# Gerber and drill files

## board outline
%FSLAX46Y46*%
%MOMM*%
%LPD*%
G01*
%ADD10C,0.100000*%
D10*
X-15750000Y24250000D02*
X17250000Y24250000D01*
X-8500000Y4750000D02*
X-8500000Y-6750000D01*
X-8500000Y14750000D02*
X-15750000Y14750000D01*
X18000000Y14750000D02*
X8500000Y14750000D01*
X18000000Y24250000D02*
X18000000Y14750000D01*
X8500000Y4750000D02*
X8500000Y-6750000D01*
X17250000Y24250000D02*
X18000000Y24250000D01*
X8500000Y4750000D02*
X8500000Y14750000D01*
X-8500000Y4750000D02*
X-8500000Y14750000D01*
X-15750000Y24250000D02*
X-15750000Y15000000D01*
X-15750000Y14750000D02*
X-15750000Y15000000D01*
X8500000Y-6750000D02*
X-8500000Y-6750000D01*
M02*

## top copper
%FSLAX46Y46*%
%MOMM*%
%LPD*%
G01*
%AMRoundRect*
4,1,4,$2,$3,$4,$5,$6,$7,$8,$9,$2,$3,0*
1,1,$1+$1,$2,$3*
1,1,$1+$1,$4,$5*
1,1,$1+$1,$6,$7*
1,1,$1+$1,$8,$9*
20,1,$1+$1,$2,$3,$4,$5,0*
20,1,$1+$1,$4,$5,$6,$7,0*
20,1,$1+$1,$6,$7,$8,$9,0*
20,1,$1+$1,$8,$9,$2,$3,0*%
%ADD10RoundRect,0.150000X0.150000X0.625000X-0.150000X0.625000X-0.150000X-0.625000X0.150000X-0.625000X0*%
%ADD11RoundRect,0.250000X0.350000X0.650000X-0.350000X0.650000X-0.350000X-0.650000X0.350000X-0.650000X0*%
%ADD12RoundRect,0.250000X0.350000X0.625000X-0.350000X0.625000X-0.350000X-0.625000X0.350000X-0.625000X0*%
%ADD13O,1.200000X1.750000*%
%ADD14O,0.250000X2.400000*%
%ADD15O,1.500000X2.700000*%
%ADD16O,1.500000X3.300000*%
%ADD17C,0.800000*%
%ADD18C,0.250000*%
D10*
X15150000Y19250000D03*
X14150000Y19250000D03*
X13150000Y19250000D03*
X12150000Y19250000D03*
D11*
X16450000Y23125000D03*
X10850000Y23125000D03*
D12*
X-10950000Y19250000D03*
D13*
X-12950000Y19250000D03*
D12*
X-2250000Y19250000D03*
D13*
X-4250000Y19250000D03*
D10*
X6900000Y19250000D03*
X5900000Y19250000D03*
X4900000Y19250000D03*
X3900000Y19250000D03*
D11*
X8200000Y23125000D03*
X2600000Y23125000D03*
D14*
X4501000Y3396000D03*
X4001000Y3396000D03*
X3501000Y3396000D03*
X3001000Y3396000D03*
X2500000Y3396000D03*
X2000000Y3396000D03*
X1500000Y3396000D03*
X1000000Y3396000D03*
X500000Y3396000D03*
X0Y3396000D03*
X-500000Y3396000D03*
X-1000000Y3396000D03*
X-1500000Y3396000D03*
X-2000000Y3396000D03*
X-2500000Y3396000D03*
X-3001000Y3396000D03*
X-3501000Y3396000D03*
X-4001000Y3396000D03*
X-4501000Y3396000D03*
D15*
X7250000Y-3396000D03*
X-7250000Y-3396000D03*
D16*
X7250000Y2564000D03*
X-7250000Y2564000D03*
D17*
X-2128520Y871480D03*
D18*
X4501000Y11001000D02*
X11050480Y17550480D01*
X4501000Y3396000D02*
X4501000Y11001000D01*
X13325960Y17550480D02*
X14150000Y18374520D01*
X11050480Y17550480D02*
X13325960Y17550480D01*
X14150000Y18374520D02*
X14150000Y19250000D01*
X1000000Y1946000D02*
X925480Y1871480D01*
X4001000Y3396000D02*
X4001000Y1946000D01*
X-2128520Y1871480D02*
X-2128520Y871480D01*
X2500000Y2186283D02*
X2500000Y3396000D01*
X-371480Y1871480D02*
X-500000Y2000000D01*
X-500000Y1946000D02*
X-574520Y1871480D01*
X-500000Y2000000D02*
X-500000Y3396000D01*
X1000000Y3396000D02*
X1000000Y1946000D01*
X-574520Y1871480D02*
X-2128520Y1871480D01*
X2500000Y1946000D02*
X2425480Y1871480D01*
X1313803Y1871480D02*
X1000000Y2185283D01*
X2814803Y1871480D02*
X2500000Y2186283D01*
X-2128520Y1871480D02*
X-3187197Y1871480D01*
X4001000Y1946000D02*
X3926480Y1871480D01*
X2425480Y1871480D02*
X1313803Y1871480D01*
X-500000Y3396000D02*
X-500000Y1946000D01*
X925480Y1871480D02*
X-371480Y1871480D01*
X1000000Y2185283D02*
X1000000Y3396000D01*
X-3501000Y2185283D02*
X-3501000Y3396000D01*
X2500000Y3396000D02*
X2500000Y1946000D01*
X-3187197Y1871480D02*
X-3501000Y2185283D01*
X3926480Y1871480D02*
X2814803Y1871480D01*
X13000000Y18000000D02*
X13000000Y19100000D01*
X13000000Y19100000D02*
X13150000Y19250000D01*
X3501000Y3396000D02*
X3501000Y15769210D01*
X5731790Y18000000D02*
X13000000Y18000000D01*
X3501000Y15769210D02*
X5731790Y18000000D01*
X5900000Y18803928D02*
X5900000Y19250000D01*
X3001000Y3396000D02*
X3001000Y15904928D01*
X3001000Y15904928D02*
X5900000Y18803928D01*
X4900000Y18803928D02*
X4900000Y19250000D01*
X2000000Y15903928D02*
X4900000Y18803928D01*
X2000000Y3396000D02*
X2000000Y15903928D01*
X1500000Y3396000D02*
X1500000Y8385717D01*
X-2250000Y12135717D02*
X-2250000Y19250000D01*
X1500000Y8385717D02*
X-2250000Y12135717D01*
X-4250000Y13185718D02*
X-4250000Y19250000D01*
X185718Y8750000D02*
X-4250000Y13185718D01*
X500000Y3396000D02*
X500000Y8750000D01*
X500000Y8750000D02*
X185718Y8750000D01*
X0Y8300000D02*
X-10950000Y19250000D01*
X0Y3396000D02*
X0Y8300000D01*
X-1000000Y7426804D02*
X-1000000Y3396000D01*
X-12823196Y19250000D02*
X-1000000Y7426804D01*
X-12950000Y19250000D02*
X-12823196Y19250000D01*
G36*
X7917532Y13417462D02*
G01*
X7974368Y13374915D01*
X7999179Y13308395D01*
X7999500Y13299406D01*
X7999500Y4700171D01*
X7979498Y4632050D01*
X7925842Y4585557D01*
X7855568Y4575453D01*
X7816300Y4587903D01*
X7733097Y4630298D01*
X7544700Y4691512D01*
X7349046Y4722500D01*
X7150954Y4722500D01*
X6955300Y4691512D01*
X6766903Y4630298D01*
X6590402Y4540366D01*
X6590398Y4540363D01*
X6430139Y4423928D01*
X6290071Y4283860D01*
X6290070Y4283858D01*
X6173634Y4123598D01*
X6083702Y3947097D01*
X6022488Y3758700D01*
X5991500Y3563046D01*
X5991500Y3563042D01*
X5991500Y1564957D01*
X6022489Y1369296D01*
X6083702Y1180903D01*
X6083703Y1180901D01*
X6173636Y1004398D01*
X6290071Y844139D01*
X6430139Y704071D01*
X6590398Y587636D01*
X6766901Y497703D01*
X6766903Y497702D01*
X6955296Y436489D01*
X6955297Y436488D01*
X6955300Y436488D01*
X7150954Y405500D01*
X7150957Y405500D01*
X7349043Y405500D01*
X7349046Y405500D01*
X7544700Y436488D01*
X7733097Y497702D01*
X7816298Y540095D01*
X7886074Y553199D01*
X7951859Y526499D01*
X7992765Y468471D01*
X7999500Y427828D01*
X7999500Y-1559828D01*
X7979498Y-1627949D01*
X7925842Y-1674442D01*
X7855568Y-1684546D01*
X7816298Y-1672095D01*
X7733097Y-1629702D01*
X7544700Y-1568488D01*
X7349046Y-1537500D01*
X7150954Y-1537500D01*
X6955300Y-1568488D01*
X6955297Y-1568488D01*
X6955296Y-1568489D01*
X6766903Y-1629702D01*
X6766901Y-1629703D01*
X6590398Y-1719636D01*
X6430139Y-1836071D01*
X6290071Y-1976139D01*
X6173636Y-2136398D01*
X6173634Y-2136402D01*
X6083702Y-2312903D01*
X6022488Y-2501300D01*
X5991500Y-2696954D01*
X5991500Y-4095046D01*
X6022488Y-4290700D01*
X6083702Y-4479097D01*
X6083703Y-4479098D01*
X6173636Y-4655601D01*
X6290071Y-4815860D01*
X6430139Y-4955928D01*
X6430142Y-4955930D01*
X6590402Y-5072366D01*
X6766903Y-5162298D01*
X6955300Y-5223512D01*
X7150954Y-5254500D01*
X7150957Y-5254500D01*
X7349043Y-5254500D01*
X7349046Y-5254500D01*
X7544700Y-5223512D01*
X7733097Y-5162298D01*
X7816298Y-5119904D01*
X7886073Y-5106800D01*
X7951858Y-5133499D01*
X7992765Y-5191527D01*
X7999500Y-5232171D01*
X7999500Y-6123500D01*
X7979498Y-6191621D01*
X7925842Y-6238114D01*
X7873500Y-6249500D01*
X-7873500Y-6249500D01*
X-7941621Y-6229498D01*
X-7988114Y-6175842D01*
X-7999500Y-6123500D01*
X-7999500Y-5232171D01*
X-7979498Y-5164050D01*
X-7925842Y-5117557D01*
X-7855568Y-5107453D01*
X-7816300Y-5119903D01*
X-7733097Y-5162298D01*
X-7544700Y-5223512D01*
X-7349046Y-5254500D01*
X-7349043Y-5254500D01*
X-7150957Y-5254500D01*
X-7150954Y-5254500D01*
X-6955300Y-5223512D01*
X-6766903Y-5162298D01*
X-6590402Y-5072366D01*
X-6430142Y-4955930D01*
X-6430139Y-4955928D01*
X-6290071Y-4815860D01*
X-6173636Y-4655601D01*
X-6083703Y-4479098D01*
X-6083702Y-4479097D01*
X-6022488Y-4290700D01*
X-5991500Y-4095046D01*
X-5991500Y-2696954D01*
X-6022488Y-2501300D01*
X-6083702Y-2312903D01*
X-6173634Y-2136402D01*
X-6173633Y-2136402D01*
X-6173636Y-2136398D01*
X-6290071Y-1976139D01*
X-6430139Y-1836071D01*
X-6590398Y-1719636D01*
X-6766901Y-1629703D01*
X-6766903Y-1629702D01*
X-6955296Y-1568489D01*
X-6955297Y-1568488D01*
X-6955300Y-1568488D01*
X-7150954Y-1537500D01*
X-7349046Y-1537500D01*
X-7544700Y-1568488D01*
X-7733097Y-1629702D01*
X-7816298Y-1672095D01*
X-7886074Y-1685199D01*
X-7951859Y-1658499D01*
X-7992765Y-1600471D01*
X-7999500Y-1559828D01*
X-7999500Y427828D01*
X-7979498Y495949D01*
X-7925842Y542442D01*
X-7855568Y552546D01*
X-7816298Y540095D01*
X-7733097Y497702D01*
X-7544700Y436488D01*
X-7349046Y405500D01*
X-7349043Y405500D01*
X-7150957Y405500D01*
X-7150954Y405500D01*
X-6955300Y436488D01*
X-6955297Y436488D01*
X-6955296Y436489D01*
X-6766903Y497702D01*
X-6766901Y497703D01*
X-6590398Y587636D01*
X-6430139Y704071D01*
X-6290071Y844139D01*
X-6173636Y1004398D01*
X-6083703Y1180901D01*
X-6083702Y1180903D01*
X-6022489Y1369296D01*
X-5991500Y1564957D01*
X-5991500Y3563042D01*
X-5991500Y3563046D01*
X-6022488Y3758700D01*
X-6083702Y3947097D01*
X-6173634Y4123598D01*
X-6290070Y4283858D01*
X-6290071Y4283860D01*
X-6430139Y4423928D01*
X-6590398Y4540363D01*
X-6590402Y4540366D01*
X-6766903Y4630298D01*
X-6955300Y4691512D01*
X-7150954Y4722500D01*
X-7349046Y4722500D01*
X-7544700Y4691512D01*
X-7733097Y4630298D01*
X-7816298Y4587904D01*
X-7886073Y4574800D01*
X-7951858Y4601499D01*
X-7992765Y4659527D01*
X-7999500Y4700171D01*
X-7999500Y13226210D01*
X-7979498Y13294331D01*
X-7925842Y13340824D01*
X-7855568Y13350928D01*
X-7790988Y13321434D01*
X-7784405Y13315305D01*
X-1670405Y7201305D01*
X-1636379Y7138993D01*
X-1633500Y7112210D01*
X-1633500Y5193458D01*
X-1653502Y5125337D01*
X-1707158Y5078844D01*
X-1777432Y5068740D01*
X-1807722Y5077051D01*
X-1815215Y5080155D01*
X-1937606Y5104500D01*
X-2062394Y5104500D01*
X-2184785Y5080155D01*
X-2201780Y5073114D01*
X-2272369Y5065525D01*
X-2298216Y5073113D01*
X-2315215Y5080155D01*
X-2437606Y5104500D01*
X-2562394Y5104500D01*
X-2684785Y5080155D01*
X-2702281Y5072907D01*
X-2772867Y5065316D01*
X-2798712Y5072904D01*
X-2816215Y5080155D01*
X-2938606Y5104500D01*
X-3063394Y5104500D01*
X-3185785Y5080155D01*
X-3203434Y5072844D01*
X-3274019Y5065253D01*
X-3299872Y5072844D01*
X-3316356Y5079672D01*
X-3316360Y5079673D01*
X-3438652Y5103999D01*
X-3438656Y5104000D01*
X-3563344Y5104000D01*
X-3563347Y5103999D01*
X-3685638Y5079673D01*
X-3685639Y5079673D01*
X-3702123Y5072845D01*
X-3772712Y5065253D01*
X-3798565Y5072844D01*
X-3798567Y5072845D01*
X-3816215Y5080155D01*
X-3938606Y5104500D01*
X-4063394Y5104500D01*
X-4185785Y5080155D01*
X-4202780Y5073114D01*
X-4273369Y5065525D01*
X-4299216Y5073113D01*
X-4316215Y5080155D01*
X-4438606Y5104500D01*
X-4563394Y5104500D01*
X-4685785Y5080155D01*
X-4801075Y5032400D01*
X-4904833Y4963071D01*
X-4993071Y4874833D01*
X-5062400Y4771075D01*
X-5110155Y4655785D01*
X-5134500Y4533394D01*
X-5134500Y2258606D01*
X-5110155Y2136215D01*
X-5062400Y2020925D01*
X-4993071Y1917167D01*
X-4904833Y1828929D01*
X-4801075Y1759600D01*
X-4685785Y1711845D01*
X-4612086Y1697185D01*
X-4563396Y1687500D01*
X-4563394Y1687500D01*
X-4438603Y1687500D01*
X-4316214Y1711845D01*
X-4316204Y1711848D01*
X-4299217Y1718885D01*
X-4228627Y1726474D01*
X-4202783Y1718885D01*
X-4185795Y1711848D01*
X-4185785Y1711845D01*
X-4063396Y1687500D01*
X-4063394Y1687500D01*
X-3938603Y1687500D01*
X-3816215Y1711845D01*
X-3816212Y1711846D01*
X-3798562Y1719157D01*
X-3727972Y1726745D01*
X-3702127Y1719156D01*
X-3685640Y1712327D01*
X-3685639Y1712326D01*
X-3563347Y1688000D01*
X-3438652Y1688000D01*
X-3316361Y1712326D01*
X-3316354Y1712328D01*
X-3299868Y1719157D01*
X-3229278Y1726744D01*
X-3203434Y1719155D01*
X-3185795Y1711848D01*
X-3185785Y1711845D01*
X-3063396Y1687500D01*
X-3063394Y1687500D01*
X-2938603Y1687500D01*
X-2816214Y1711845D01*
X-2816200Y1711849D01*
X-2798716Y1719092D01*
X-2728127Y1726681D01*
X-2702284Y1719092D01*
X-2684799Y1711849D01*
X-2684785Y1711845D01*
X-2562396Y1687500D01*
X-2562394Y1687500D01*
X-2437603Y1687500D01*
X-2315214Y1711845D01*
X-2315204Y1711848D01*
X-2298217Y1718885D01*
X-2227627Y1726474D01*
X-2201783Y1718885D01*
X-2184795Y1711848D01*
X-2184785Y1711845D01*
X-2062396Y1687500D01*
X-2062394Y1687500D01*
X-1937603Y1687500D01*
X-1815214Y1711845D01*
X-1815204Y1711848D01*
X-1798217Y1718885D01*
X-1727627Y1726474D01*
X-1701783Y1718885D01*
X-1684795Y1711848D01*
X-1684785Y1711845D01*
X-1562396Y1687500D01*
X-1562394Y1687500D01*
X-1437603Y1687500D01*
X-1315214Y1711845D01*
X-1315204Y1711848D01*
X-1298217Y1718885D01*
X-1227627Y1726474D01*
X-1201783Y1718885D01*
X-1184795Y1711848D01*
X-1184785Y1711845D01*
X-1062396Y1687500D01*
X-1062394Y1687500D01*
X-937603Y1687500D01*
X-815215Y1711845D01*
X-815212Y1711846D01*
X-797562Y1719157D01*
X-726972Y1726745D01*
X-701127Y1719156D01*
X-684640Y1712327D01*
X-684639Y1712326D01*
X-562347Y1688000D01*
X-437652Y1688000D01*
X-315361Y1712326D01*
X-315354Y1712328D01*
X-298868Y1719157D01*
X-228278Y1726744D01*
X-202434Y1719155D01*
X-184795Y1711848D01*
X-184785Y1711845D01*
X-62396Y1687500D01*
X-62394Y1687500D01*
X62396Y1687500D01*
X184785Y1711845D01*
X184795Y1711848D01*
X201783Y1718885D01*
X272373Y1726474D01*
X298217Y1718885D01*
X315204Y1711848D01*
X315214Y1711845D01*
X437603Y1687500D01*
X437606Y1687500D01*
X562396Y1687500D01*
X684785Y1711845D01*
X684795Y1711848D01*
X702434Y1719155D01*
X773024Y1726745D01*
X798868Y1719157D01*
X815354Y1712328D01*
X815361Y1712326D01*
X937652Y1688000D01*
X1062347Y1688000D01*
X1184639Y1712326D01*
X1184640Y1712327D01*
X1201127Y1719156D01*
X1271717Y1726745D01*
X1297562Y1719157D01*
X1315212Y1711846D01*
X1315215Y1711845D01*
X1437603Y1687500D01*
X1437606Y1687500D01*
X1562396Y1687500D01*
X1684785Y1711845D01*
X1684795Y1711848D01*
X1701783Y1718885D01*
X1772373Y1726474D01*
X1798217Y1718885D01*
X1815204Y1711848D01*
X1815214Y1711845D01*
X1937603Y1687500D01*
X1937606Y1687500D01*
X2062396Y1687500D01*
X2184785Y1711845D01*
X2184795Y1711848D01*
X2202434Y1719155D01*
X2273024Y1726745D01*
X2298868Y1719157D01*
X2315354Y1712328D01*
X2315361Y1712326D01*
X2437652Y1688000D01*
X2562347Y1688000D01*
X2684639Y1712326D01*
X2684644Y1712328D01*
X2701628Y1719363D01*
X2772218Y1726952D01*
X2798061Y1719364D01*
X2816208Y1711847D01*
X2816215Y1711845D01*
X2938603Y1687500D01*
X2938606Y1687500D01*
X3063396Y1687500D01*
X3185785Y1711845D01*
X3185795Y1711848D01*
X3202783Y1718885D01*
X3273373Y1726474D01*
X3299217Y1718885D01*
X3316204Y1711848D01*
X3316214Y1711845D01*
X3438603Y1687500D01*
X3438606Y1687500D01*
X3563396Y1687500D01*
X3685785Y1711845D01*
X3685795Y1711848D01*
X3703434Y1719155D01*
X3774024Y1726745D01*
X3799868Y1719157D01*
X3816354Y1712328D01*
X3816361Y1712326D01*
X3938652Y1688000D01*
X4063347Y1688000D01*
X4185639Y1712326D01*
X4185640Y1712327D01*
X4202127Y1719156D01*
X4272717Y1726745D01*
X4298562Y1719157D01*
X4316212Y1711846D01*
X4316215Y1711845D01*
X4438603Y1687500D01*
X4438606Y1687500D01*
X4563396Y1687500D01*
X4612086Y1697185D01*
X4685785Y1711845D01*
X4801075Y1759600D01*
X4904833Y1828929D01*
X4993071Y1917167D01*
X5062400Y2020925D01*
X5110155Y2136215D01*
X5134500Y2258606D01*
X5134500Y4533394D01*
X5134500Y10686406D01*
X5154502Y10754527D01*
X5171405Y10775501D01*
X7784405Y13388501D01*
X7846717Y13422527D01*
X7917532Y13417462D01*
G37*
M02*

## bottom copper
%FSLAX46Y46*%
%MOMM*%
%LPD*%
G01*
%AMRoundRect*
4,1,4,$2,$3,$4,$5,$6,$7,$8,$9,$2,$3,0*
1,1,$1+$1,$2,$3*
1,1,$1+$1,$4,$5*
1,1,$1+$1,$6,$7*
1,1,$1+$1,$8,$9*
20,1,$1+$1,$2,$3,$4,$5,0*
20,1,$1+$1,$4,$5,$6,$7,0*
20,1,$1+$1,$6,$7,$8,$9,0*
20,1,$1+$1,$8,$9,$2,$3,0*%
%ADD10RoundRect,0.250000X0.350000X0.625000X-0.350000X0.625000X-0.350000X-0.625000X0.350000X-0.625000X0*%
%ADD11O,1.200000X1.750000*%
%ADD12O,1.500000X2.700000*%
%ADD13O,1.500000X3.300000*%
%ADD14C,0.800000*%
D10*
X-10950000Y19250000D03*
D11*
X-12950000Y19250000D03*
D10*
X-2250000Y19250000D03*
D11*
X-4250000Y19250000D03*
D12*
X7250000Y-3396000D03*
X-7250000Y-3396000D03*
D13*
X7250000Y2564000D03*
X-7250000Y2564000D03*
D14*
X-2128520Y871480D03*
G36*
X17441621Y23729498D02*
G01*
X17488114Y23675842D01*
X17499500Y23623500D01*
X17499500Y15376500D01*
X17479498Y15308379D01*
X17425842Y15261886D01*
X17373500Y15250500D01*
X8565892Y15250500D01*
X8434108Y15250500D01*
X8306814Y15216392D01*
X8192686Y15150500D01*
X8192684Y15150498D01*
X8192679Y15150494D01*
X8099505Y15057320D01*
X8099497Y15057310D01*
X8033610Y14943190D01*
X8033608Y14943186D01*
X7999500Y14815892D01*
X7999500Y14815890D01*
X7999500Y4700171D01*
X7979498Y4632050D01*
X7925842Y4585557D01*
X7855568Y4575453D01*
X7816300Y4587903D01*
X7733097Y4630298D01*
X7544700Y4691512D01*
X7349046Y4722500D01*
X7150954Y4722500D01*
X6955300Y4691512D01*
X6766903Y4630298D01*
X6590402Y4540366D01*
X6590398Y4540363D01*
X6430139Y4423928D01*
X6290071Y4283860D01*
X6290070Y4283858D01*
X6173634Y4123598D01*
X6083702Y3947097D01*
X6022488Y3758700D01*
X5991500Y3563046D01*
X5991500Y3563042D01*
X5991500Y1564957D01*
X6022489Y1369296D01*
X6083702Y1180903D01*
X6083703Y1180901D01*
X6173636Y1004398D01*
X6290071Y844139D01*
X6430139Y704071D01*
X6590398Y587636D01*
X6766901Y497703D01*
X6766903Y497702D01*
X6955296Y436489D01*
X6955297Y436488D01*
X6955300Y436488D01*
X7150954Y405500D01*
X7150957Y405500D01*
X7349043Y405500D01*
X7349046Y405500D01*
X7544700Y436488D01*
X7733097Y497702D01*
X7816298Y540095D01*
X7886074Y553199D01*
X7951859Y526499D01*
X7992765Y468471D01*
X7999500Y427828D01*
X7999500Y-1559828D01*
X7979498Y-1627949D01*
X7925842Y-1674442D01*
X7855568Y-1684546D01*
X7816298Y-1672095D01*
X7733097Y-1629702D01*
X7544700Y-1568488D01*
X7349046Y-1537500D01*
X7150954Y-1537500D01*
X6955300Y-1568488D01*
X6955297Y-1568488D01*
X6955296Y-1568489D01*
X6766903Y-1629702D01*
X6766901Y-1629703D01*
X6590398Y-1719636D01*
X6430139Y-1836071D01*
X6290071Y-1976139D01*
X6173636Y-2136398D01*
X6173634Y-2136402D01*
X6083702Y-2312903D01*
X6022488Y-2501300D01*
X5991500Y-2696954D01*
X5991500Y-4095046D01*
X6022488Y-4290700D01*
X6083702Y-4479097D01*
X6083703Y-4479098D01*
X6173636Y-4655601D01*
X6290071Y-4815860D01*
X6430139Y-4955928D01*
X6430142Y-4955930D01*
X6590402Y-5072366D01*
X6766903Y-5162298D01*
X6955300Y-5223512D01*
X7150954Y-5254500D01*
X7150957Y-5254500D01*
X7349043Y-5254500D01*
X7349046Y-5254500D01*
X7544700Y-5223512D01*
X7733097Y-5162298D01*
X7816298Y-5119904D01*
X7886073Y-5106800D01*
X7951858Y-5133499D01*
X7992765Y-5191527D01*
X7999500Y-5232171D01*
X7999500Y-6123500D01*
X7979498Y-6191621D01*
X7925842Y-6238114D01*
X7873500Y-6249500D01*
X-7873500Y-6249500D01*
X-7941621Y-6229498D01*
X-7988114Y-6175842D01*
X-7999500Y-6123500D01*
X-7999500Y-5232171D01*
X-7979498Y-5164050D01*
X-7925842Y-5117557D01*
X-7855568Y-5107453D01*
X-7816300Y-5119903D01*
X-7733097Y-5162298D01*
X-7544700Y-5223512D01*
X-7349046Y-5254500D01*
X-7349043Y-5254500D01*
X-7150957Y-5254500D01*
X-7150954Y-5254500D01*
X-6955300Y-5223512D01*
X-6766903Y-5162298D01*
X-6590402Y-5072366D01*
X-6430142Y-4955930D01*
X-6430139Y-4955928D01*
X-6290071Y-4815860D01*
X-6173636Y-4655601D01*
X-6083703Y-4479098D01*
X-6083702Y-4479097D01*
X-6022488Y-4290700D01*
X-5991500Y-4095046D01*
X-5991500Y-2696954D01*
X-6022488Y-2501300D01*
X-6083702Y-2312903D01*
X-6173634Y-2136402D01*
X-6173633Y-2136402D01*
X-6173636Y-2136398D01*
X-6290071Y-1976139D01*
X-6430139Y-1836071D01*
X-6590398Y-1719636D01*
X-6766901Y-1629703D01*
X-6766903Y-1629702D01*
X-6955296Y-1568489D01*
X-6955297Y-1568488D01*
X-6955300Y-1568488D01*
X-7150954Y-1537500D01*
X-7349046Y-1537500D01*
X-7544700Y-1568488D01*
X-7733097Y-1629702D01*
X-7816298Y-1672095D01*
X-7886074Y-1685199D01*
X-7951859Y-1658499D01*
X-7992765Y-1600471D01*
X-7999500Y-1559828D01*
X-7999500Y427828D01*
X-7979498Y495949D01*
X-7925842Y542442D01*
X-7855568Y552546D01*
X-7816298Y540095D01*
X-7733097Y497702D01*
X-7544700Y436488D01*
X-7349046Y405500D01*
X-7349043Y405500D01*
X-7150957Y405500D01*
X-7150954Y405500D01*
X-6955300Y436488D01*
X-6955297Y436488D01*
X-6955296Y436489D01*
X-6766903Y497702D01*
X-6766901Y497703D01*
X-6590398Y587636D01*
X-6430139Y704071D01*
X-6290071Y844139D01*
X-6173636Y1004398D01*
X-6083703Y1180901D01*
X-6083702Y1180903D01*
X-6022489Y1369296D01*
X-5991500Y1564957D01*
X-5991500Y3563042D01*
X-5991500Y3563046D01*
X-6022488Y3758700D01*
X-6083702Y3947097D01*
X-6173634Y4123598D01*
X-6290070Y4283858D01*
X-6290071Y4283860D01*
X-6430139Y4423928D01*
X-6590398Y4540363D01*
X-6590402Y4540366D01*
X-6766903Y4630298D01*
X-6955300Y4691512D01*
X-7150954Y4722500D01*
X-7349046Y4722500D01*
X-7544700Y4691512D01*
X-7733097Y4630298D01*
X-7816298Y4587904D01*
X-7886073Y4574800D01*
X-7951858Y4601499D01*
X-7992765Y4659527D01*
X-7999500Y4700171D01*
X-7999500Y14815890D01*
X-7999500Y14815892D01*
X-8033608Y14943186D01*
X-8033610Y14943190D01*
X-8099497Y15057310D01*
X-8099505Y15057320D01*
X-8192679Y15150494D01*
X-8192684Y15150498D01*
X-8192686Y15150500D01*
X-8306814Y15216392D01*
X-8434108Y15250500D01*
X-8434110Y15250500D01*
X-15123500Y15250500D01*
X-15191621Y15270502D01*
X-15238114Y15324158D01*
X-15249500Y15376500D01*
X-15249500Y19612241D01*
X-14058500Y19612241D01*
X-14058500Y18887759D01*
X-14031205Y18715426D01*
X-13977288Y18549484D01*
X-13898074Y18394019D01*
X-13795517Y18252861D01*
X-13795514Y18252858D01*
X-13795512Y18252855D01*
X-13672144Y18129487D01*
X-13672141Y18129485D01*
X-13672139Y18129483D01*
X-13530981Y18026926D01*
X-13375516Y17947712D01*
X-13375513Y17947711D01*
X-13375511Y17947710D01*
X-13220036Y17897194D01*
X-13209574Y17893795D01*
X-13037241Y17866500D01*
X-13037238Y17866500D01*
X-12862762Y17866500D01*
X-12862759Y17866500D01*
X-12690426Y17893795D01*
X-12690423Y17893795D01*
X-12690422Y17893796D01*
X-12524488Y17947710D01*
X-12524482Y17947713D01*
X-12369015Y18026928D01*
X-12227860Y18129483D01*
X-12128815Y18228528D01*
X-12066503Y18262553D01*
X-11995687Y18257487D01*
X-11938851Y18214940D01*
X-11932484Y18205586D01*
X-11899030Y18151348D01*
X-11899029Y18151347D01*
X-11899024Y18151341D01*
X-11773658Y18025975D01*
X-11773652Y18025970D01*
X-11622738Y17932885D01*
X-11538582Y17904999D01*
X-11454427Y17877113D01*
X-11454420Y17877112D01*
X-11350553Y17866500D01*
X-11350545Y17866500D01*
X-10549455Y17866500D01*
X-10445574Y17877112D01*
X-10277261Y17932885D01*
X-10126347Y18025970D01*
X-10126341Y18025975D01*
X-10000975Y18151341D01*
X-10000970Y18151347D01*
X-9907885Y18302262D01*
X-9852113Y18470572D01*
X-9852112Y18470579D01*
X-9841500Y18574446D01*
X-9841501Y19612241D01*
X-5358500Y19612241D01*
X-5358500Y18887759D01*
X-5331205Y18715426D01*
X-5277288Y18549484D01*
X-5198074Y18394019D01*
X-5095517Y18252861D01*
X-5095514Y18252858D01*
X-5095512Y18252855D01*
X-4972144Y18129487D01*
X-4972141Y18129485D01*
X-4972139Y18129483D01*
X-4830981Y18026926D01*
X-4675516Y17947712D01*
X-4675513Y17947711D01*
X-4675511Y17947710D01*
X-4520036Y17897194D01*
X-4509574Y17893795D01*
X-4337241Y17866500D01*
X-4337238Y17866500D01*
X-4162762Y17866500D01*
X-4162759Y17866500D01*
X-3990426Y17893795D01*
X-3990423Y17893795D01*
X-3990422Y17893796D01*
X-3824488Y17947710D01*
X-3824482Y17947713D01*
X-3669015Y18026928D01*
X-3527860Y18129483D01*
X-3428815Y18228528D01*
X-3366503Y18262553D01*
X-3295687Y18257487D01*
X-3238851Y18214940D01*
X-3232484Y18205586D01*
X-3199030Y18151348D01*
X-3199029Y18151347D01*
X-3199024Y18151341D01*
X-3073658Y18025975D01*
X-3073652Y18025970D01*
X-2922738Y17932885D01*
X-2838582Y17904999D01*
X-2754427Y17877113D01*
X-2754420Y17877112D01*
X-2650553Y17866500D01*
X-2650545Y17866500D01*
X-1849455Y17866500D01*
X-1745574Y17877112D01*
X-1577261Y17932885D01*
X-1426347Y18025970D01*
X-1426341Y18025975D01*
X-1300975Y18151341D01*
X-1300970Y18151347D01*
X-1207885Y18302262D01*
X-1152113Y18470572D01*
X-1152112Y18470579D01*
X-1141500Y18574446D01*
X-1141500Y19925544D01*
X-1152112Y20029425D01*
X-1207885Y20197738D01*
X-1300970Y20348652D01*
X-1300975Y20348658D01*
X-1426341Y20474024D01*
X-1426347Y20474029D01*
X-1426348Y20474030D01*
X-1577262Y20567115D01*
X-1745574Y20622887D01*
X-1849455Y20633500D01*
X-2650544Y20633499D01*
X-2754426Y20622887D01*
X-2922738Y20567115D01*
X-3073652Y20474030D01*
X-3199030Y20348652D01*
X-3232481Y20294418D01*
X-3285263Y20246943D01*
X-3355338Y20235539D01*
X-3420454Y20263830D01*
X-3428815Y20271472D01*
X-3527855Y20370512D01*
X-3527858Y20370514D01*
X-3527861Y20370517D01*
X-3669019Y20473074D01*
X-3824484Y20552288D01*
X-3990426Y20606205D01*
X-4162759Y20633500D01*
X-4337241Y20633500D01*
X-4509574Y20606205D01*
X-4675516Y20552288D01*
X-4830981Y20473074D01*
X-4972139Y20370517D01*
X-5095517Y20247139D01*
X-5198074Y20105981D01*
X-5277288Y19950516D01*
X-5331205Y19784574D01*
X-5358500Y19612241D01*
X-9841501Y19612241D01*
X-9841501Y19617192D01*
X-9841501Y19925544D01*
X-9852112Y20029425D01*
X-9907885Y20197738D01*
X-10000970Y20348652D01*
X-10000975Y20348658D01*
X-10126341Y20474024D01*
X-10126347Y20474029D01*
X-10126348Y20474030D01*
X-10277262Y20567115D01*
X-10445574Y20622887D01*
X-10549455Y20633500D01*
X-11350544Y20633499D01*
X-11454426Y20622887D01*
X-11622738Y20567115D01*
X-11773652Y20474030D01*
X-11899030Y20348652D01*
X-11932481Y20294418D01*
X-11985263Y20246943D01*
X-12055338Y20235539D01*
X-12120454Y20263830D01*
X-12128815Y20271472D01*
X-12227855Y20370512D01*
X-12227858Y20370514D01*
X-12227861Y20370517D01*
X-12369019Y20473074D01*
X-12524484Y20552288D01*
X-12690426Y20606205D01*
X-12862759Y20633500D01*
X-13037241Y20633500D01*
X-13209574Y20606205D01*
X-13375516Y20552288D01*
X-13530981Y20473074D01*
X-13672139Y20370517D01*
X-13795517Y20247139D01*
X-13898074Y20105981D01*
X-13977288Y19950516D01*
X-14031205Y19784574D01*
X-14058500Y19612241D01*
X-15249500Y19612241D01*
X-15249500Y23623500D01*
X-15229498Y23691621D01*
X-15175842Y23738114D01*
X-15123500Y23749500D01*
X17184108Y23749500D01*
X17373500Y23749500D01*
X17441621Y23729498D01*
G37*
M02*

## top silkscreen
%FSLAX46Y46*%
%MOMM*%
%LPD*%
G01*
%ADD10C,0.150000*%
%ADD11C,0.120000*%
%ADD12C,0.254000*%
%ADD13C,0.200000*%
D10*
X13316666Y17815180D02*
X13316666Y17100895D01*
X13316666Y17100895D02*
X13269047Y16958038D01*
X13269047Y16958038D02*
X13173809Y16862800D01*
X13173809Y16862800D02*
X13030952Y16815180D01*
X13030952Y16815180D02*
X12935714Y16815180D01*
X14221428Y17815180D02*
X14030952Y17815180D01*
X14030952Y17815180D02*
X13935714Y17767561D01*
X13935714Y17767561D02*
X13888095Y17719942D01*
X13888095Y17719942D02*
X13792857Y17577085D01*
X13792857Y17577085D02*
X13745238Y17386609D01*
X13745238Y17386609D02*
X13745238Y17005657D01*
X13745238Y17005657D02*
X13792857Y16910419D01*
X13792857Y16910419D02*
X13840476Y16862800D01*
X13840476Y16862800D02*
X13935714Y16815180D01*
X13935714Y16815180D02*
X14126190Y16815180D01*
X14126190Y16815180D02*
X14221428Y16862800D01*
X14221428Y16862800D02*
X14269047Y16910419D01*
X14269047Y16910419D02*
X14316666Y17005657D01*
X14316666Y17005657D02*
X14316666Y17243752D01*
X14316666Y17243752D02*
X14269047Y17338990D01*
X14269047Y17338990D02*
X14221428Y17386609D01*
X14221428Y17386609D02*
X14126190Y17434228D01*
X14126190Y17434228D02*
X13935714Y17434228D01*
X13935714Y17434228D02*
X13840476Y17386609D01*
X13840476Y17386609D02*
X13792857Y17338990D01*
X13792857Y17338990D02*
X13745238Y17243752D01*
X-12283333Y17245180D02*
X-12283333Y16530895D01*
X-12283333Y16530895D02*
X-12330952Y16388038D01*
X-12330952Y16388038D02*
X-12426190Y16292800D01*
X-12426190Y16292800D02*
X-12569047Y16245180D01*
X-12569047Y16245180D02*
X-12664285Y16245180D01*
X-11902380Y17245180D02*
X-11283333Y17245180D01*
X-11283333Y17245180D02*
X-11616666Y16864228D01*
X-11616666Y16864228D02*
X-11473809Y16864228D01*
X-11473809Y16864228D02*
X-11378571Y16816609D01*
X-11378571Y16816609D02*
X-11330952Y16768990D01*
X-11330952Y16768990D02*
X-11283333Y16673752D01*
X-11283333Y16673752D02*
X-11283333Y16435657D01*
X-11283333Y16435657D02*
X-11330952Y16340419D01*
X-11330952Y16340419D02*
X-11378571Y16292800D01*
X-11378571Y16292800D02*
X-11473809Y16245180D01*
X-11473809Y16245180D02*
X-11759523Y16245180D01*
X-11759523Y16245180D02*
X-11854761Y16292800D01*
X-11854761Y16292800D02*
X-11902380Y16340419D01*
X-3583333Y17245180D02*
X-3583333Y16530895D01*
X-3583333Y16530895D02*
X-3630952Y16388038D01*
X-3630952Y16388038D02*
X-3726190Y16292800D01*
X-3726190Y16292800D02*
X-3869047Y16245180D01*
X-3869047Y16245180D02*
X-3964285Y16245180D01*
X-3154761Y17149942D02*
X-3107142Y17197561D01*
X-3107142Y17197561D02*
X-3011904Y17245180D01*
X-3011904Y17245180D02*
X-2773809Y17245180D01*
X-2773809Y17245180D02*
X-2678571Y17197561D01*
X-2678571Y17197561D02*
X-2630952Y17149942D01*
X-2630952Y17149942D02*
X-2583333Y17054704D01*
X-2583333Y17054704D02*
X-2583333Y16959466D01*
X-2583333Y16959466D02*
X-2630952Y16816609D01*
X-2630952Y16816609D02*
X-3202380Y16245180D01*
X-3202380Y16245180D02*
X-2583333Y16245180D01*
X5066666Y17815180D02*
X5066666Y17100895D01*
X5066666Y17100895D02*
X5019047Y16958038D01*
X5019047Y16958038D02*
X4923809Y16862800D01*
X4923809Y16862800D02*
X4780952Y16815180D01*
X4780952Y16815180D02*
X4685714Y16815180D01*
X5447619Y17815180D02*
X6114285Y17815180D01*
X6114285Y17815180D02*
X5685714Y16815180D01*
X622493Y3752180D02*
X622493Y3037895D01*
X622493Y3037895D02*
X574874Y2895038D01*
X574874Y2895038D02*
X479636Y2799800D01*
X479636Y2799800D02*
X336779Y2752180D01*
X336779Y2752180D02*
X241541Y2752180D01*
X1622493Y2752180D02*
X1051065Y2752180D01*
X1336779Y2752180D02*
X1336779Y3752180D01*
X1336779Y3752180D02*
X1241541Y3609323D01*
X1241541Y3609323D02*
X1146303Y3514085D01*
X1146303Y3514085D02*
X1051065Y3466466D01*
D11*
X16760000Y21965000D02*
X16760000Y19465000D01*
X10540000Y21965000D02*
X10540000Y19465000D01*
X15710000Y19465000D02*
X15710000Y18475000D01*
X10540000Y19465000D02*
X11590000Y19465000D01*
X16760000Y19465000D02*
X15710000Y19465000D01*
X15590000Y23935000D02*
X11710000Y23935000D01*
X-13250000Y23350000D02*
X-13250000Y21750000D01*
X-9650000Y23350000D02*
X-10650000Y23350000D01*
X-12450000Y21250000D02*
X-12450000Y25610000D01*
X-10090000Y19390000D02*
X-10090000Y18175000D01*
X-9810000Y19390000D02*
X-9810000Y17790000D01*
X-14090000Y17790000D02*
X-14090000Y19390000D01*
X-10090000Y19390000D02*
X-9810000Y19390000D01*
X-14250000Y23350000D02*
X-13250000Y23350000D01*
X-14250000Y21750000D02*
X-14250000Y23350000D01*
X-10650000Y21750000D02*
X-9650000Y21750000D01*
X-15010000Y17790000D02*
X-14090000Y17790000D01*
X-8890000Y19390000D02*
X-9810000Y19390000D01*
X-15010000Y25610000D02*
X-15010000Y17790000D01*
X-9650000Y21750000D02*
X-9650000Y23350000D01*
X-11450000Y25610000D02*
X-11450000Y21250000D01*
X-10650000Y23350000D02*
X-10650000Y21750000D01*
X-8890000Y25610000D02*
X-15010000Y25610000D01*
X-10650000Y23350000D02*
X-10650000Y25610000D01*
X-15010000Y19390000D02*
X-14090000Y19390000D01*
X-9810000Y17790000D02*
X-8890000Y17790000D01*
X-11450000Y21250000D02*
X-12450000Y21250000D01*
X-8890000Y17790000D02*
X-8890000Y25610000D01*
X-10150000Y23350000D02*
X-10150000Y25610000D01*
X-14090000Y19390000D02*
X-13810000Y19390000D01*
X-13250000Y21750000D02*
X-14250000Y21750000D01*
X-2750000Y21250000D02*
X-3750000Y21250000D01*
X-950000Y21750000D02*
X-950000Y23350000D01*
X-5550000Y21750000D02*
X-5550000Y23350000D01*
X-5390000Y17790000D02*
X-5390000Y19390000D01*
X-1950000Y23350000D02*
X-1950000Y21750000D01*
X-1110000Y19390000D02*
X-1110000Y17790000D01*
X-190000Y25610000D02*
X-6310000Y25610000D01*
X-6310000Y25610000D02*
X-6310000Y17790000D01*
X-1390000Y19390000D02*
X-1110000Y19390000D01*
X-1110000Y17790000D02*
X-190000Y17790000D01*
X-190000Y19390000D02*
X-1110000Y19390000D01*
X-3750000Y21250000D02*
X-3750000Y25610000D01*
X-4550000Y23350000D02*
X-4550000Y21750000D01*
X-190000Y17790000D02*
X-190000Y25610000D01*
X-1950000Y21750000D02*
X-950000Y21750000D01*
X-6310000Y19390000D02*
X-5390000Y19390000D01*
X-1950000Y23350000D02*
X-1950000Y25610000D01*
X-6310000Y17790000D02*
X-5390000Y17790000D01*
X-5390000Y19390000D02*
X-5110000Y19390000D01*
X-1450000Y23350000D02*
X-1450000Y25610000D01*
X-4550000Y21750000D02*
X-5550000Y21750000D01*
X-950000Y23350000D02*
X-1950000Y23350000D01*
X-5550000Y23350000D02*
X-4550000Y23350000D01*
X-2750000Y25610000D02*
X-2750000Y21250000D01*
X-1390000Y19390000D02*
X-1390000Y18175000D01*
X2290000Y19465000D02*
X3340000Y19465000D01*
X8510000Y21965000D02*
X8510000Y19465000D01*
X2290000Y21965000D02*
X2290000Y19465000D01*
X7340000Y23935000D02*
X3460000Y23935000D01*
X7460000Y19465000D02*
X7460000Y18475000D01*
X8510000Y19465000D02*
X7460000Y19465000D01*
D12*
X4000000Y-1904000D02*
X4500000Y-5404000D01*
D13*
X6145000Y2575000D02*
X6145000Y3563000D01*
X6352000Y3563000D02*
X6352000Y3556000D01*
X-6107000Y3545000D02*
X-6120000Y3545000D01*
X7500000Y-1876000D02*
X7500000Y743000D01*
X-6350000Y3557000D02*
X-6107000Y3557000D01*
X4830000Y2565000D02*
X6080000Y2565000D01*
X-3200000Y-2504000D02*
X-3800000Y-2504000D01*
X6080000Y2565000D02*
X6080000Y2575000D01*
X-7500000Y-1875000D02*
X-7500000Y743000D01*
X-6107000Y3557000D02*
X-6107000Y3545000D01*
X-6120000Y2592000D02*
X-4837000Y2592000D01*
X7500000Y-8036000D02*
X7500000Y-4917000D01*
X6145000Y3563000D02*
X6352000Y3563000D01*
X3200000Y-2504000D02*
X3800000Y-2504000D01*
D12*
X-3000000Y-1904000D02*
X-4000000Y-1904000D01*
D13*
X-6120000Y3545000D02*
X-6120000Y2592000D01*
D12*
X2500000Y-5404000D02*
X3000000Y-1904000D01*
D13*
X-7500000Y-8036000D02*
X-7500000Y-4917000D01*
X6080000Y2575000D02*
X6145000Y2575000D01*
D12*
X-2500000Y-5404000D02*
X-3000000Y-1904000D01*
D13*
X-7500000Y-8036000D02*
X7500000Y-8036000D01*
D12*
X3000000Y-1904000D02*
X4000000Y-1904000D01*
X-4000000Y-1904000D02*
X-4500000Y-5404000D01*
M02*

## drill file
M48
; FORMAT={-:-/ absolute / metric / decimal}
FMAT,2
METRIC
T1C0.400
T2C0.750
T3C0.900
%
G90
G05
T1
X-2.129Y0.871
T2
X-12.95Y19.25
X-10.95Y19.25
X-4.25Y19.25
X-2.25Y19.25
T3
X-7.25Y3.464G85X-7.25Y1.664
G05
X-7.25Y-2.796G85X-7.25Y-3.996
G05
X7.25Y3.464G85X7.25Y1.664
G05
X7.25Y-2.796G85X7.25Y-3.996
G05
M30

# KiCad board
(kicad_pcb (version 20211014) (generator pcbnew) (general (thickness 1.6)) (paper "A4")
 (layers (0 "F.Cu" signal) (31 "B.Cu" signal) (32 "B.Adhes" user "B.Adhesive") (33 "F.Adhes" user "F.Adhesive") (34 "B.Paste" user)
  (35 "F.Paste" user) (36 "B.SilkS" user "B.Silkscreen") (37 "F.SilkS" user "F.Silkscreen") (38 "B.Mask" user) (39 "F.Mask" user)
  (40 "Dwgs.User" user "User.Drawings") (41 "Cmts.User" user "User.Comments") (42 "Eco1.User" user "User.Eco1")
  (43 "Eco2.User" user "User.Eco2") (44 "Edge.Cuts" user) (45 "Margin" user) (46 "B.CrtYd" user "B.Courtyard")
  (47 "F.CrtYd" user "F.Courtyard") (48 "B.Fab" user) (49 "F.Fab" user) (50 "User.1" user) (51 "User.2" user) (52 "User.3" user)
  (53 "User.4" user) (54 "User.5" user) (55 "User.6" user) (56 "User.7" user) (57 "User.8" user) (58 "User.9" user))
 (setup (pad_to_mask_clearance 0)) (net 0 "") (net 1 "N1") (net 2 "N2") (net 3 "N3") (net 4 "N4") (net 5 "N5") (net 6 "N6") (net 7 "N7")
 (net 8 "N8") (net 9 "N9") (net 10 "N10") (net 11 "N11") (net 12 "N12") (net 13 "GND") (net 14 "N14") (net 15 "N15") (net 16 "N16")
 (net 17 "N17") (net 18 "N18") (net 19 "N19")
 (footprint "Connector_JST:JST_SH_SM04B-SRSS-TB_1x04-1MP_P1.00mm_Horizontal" (layer "F.Cu") (at 13.65 -21.25 180)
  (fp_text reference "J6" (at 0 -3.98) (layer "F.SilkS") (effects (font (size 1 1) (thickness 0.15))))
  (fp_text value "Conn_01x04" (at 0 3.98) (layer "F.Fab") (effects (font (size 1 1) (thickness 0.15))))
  (fp_line (start -3.11 0.715) (end -3.11 -1.785) (layer "F.SilkS") (width 0.12))
  (fp_line (start 3.11 0.715) (end 3.11 -1.785) (layer "F.SilkS") (width 0.12))
  (fp_line (start -2.06 -1.785) (end -2.06 -2.775) (layer "F.SilkS") (width 0.12))
  (fp_line (start 3.11 -1.785) (end 2.06 -1.785) (layer "F.SilkS") (width 0.12))
  (fp_line (start -3.11 -1.785) (end -2.06 -1.785) (layer "F.SilkS") (width 0.12))
  (fp_line (start -1.94 2.685) (end 1.94 2.685) (layer "F.SilkS") (width 0.12))
  (pad "1" smd roundrect (at -1.5 -2 180) (size 0.6 1.55) (layers "F.Cu" "F.Paste" "F.Mask") (roundrect_rratio 0.25) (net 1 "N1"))
  (pad "2" smd roundrect (at -0.5 -2 180) (size 0.6 1.55) (layers "F.Cu" "F.Paste" "F.Mask") (roundrect_rratio 0.25) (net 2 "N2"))
  (pad "3" smd roundrect (at 0.5 -2 180) (size 0.6 1.55) (layers "F.Cu" "F.Paste" "F.Mask") (roundrect_rratio 0.25) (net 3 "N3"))
  (pad "4" smd roundrect (at 1.5 -2 180) (size 0.6 1.55) (layers "F.Cu" "F.Paste" "F.Mask") (roundrect_rratio 0.25) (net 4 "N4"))
  (pad "MP" smd roundrect (at -2.8 1.875 180) (size 1.2 1.8) (layers "F.Cu" "F.Paste" "F.Mask") (roundrect_rratio 0.2083333333))
  (pad "MP" smd roundrect (at 2.8 1.875 180) (size 1.2 1.8) (layers "F.Cu" "F.Paste" "F.Mask") (roundrect_rratio 0.2083333333)))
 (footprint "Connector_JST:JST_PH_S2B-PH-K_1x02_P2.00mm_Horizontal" (layer "F.Cu") (at -10.95 -19.25 180)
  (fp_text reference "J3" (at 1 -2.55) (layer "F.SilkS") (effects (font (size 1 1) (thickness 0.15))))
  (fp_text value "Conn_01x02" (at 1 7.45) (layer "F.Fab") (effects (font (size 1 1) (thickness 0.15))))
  (fp_line (start 2.3 4.1) (end 2.3 2.5) (layer "F.SilkS") (width 0.12))
  (fp_line (start -1.3 4.1) (end -0.3 4.1) (layer "F.SilkS") (width 0.12))
  (fp_line (start 1.5 2) (end 1.5 6.36) (layer "F.SilkS") (width 0.12))
  (fp_line (start -0.86 0.14) (end -0.86 -1.075) (layer "F.SilkS") (width 0.12))
  (fp_line (start -1.14 0.14) (end -1.14 -1.46) (layer "F.SilkS") (width 0.12))
  (fp_line (start 3.14 -1.46) (end 3.14 0.14) (layer "F.SilkS") (width 0.12))
  (fp_line (start -0.86 0.14) (end -1.14 0.14) (layer "F.SilkS") (width 0.12))
  (fp_line (start 3.3 4.1) (end 2.3 4.1) (layer "F.SilkS") (width 0.12))
  (fp_line (start 3.3 2.5) (end 3.3 4.1) (layer "F.SilkS") (width 0.12))
  (fp_line (start -0.3 2.5) (end -1.3 2.5) (layer "F.SilkS") (width 0.12))
  (fp_line (start 4.06 -1.46) (end 3.14 -1.46) (layer "F.SilkS") (width 0.12))
  (fp_line (start -2.06 0.14) (end -1.14 0.14) (layer "F.SilkS") (width 0.12))
  (fp_line (start 4.06 6.36) (end 4.06 -1.46) (layer "F.SilkS") (width 0.12))
  (fp_line (start -1.3 2.5) (end -1.3 4.1) (layer "F.SilkS") (width 0.12))
  (fp_line (start 0.5 6.36) (end 0.5 2) (layer "F.SilkS") (width 0.12))
  (fp_line (start -0.3 4.1) (end -0.3 2.5) (layer "F.SilkS") (width 0.12))
  (fp_line (start -2.06 6.36) (end 4.06 6.36) (layer "F.SilkS") (width 0.12))
  (fp_line (start -0.3 4.1) (end -0.3 6.36) (layer "F.SilkS") (width 0.12))
  (fp_line (start 4.06 0.14) (end 3.14 0.14) (layer "F.SilkS") (width 0.12))
  (fp_line (start -1.14 -1.46) (end -2.06 -1.46) (layer "F.SilkS") (width 0.12))
  (fp_line (start 0.5 2) (end 1.5 2) (layer "F.SilkS") (width 0.12))
  (fp_line (start -2.06 -1.46) (end -2.06 6.36) (layer "F.SilkS") (width 0.12))
  (fp_line (start -0.8 4.1) (end -0.8 6.36) (layer "F.SilkS") (width 0.12))
  (fp_line (start 3.14 0.14) (end 2.86 0.14) (layer "F.SilkS") (width 0.12))
  (fp_line (start 2.3 2.5) (end 3.3 2.5) (layer "F.SilkS") (width 0.12))
  (pad "1" thru_hole roundrect (at 0 0 180) (size 1.2 1.75) (drill 0.75) (layers *.Cu *.Mask) (roundrect_rratio 0.2083333333) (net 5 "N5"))
  (pad "2" thru_hole oval (at 2 0 180) (size 1.2 1.75) (drill 0.75) (layers *.Cu *.Mask) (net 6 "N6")))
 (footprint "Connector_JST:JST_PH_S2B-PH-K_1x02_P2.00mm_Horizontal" (layer "F.Cu") (at -2.25 -19.25 180)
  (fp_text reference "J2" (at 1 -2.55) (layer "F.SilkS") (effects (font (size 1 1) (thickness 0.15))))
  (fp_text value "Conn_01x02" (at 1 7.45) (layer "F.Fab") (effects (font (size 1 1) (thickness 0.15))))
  (fp_line (start 0.5 2) (end 1.5 2) (layer "F.SilkS") (width 0.12))
  (fp_line (start -1.3 2.5) (end -1.3 4.1) (layer "F.SilkS") (width 0.12))
  (fp_line (start 3.3 2.5) (end 3.3 4.1) (layer "F.SilkS") (width 0.12))
  (fp_line (start 3.14 -1.46) (end 3.14 0.14) (layer "F.SilkS") (width 0.12))
  (fp_line (start -0.3 4.1) (end -0.3 2.5) (layer "F.SilkS") (width 0.12))
  (fp_line (start -1.14 0.14) (end -1.14 -1.46) (layer "F.SilkS") (width 0.12))
  (fp_line (start -2.06 6.36) (end 4.06 6.36) (layer "F.SilkS") (width 0.12))
  (fp_line (start 4.06 6.36) (end 4.06 -1.46) (layer "F.SilkS") (width 0.12))
  (fp_line (start -0.86 0.14) (end -1.14 0.14) (layer "F.SilkS") (width 0.12))
  (fp_line (start -1.14 -1.46) (end -2.06 -1.46) (layer "F.SilkS") (width 0.12))
  (fp_line (start -2.06 0.14) (end -1.14 0.14) (layer "F.SilkS") (width 0.12))
  (fp_line (start 1.5 2) (end 1.5 6.36) (layer "F.SilkS") (width 0.12))
  (fp_line (start 2.3 4.1) (end 2.3 2.5) (layer "F.SilkS") (width 0.12))
  (fp_line (start -2.06 -1.46) (end -2.06 6.36) (layer "F.SilkS") (width 0.12))
  (fp_line (start -0.3 2.5) (end -1.3 2.5) (layer "F.SilkS") (width 0.12))
  (fp_line (start 4.06 0.14) (end 3.14 0.14) (layer "F.SilkS") (width 0.12))
  (fp_line (start -0.3 4.1) (end -0.3 6.36) (layer "F.SilkS") (width 0.12))
  (fp_line (start 4.06 -1.46) (end 3.14 -1.46) (layer "F.SilkS") (width 0.12))
  (fp_line (start 3.14 0.14) (end 2.86 0.14) (layer "F.SilkS") (width 0.12))
  (fp_line (start -0.8 4.1) (end -0.8 6.36) (layer "F.SilkS") (width 0.12))
  (fp_line (start 2.3 2.5) (end 3.3 2.5) (layer "F.SilkS") (width 0.12))
  (fp_line (start -1.3 4.1) (end -0.3 4.1) (layer "F.SilkS") (width 0.12))
  (fp_line (start 3.3 4.1) (end 2.3 4.1) (layer "F.SilkS") (width 0.12))
  (fp_line (start 0.5 6.36) (end 0.5 2) (layer "F.SilkS") (width 0.12))
  (fp_line (start -0.86 0.14) (end -0.86 -1.075) (layer "F.SilkS") (width 0.12))
  (pad "1" thru_hole roundrect (at 0 0 180) (size 1.2 1.75) (drill 0.75) (layers *.Cu *.Mask) (roundrect_rratio 0.2083333333) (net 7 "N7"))
  (pad "2" thru_hole oval (at 2 0 180) (size 1.2 1.75) (drill 0.75) (layers *.Cu *.Mask) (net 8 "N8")))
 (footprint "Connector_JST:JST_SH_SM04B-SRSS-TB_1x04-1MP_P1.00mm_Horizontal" (layer "F.Cu") (at 5.4 -21.25 180)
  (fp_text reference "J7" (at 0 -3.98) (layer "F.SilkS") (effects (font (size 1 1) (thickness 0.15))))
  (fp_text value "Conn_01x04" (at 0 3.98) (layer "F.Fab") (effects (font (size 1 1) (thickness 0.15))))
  (fp_line (start 3.11 -1.785) (end 2.06 -1.785) (layer "F.SilkS") (width 0.12))
  (fp_line (start -3.11 0.715) (end -3.11 -1.785) (layer "F.SilkS") (width 0.12))
  (fp_line (start 3.11 0.715) (end 3.11 -1.785) (layer "F.SilkS") (width 0.12))
  (fp_line (start -1.94 2.685) (end 1.94 2.685) (layer "F.SilkS") (width 0.12))
  (fp_line (start -2.06 -1.785) (end -2.06 -2.775) (layer "F.SilkS") (width 0.12))
  (fp_line (start -3.11 -1.785) (end -2.06 -1.785) (layer "F.SilkS") (width 0.12))
  (pad "1" smd roundrect (at -1.5 -2 180) (size 0.6 1.55) (layers "F.Cu" "F.Paste" "F.Mask") (roundrect_rratio 0.25) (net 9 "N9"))
  (pad "2" smd roundrect (at -0.5 -2 180) (size 0.6 1.55) (layers "F.Cu" "F.Paste" "F.Mask") (roundrect_rratio 0.25) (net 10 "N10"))
  (pad "3" smd roundrect (at 0.5 -2 180) (size 0.6 1.55) (layers "F.Cu" "F.Paste" "F.Mask") (roundrect_rratio 0.25) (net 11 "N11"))
  (pad "4" smd roundrect (at 1.5 -2 180) (size 0.6 1.55) (layers "F.Cu" "F.Paste" "F.Mask") (roundrect_rratio 0.25) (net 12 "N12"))
  (pad "MP" smd roundrect (at -2.8 1.875 180) (size 1.2 1.8) (layers "F.Cu" "F.Paste" "F.Mask") (roundrect_rratio 0.2083333333))
  (pad "MP" smd roundrect (at 2.8 1.875 180) (size 1.2 1.8) (layers "F.Cu" "F.Paste" "F.Mask") (roundrect_rratio 0.2083333333)))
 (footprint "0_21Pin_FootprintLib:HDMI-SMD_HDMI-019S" (layer "F.Cu") (at 0 0)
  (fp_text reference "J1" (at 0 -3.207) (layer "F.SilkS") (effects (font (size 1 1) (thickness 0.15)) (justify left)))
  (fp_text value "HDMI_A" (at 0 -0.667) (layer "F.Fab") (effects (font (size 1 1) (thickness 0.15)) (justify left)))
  (fp_line (start 4 1.904) (end 4.5 5.404) (layer "F.SilkS") (width 0.254))
  (fp_line (start 6.145 -2.575) (end 6.145 -3.563) (layer "F.SilkS") (width 0.2))
  (fp_line (start 6.352 -3.563) (end 6.352 -3.556) (layer "F.SilkS") (width 0.2))
  (fp_line (start -6.107 -3.545) (end -6.12 -3.545) (layer "F.SilkS") (width 0.2))
  (fp_line (start 7.5 1.876) (end 7.5 -0.743) (layer "F.SilkS") (width 0.2))
  (fp_line (start -6.35 -3.557) (end -6.107 -3.557) (layer "F.SilkS") (width 0.2))
  (fp_line (start 4.83 -2.565) (end 6.08 -2.565) (layer "F.SilkS") (width 0.2))
  (fp_line (start -3.2 2.504) (end -3.8 2.504) (layer "F.SilkS") (width 0.2))
  (fp_line (start 6.08 -2.565) (end 6.08 -2.575) (layer "F.SilkS") (width 0.2))
  (fp_line (start -7.5 1.875) (end -7.5 -0.743) (layer "F.SilkS") (width 0.2))
  (fp_line (start -6.107 -3.557) (end -6.107 -3.545) (layer "F.SilkS") (width 0.2))
  (fp_line (start -6.12 -2.592) (end -4.837 -2.592) (layer "F.SilkS") (width 0.2))
  (fp_line (start 7.5 8.036) (end 7.5 4.917) (layer "F.SilkS") (width 0.2))
  (fp_line (start 6.145 -3.563) (end 6.352 -3.563) (layer "F.SilkS") (width 0.2))
  (fp_line (start 3.2 2.504) (end 3.8 2.504) (layer "F.SilkS") (width 0.2))
  (fp_line (start -3 1.904) (end -4 1.904) (layer "F.SilkS") (width 0.254))
  (fp_line (start -6.12 -3.545) (end -6.12 -2.592) (layer "F.SilkS") (width 0.2))
  (fp_line (start 2.5 5.404) (end 3 1.904) (layer "F.SilkS") (width 0.254))
  (fp_line (start -7.5 8.036) (end -7.5 4.917) (layer "F.SilkS") (width 0.2))
  (fp_line (start 6.08 -2.575) (end 6.145 -2.575) (layer "F.SilkS") (width 0.2))
  (fp_line (start -2.5 5.404) (end -3 1.904) (layer "F.SilkS") (width 0.254))
  (fp_line (start -7.5 8.036) (end 7.5 8.036) (layer "F.SilkS") (width 0.2))
  (fp_line (start 3 1.904) (end 4 1.904) (layer "F.SilkS") (width 0.254))
  (fp_line (start -4 1.904) (end -4.5 5.404) (layer "F.SilkS") (width 0.254))
  (pad "1" smd oval (at 4.501 -3.396) (size 0.25 2.4) (layers "F.Cu" "F.Paste" "F.Mask") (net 2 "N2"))
  (pad "2" smd oval (at 4.001 -3.396) (size 0.25 2.4) (layers "F.Cu" "F.Paste" "F.Mask") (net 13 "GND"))
  (pad "3" smd oval (at 3.501 -3.396) (size 0.25 2.4) (layers "F.Cu" "F.Paste" "F.Mask") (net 3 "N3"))
  (pad "4" smd oval (at 3.001 -3.396) (size 0.25 2.4) (layers "F.Cu" "F.Paste" "F.Mask") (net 10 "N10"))
  (pad "5" smd oval (at 2.5 -3.396) (size 0.25 2.4) (layers "F.Cu" "F.Paste" "F.Mask") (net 13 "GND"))
  (pad "6" smd oval (at 2 -3.396) (size 0.25 2.4) (layers "F.Cu" "F.Paste" "F.Mask") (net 11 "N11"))
  (pad "7" smd oval (at 1.5 -3.396) (size 0.25 2.4) (layers "F.Cu" "F.Paste" "F.Mask") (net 7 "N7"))
  (pad "8" smd oval (at 1 -3.396) (size 0.25 2.4) (layers "F.Cu" "F.Paste" "F.Mask") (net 13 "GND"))
  (pad "9" smd oval (at 0.5 -3.396) (size 0.25 2.4) (layers "F.Cu" "F.Paste" "F.Mask") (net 8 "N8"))
  (pad "10" smd oval (at 0 -3.396) (size 0.25 2.4) (layers "F.Cu" "F.Paste" "F.Mask") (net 5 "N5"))
  (pad "11" smd oval (at -0.5 -3.396) (size 0.25 2.4) (layers "F.Cu" "F.Paste" "F.Mask") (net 13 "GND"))
  (pad "12" smd oval (at -1 -3.396) (size 0.25 2.4) (layers "F.Cu" "F.Paste" "F.Mask") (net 6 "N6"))
  (pad "13" smd oval (at -1.5 -3.396) (size 0.25 2.4) (layers "F.Cu" "F.Paste" "F.Mask") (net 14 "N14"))
  (pad "14" smd oval (at -2 -3.396) (size 0.25 2.4) (layers "F.Cu" "F.Paste" "F.Mask") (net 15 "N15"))
  (pad "15" smd oval (at -2.5 -3.396) (size 0.25 2.4) (layers "F.Cu" "F.Paste" "F.Mask") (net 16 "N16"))
  (pad "16" smd oval (at -3.001 -3.396) (size 0.25 2.4) (layers "F.Cu" "F.Paste" "F.Mask") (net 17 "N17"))
  (pad "17" smd oval (at -3.501 -3.396) (size 0.25 2.4) (layers "F.Cu" "F.Paste" "F.Mask") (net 13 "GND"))
  (pad "18" smd oval (at -4.001 -3.396) (size 0.25 2.4) (layers "F.Cu" "F.Paste" "F.Mask") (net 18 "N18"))
  (pad "19" smd oval (at -4.501 -3.396) (size 0.25 2.4) (layers "F.Cu" "F.Paste" "F.Mask") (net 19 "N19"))
  (pad "20" thru_hole oval (at 7.25 3.396) (size 1.5 2.7) (drill oval 0.9 2.1) (layers *.Cu *.Mask))
  (pad "21" thru_hole oval (at -7.25 3.396) (size 1.5 2.7) (drill oval 0.9 2.1) (layers *.Cu *.Mask))
  (pad "22" thru_hole oval (at 7.25 -2.564) (size 1.5 3.3) (drill oval 0.9 2.7) (layers *.Cu *.Mask))
  (pad "23" thru_hole oval (at -7.25 -2.564) (size 1.5 3.3) (drill oval 0.9 2.7) (layers *.Cu *.Mask)))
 (gr_line (start -15.75 -24.25) (end 17.25 -24.25) (layer "Edge.Cuts") (width 0.1))
 (gr_line (start -8.5 -4.75) (end -8.5 6.75) (layer "Edge.Cuts") (width 0.1))
 (gr_line (start -8.5 -14.75) (end -15.75 -14.75) (layer "Edge.Cuts") (width 0.1))
 (gr_line (start 18 -14.75) (end 8.5 -14.75) (layer "Edge.Cuts") (width 0.1))
 (gr_line (start 18 -24.25) (end 18 -14.75) (layer "Edge.Cuts") (width 0.1))
 (gr_line (start 8.5 -4.75) (end 8.5 6.75) (layer "Edge.Cuts") (width 0.1))
 (gr_line (start 17.25 -24.25) (end 18 -24.25) (layer "Edge.Cuts") (width 0.1))
 (gr_line (start 8.5 -4.75) (end 8.5 -14.75) (layer "Edge.Cuts") (width 0.1))
 (gr_line (start -8.5 -4.75) (end -8.5 -14.75) (layer "Edge.Cuts") (width 0.1))
 (gr_line (start -15.75 -24.25) (end -15.75 -15) (layer "Edge.Cuts") (width 0.1))
 (gr_line (start -15.75 -14.75) (end -15.75 -15) (layer "Edge.Cuts") (width 0.1))
 (gr_line (start 8.5 6.75) (end -8.5 6.75) (layer "Edge.Cuts") (width 0.1))
 (segment (start 4.501 -11.001) (end 11.05048 -17.55048) (width 0.25) (layer "F.Cu") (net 2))
 (segment (start 4.501 -3.396) (end 4.501 -11.001) (width 0.25) (layer "F.Cu") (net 2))
 (segment (start 13.32596 -17.55048) (end 14.15 -18.37452) (width 0.25) (layer "F.Cu") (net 2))
 (segment (start 11.05048 -17.55048) (end 13.32596 -17.55048) (width 0.25) (layer "F.Cu") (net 2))
 (segment (start 14.15 -18.37452) (end 14.15 -19.25) (width 0.25) (layer "F.Cu") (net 2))
 (segment (start 1 -1.946) (end 0.92548 -1.87148) (width 0.25) (layer "F.Cu") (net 13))
 (segment (start 4.001 -3.396) (end 4.001 -1.946) (width 0.25) (layer "F.Cu") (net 13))
 (segment (start -2.12852 -1.87148) (end -2.12852 -0.87148) (width 0.25) (layer "F.Cu") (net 13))
 (segment (start 2.5 -2.186283) (end 2.5 -3.396) (width 0.25) (layer "F.Cu") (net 13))
 (segment (start -0.37148 -1.87148) (end -0.5 -2) (width 0.25) (layer "F.Cu") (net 13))
 (segment (start -0.5 -1.946) (end -0.57452 -1.87148) (width 0.25) (layer "F.Cu") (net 13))
 (segment (start -0.5 -2) (end -0.5 -3.396) (width 0.25) (layer "F.Cu") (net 13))
 (segment (start 1 -3.396) (end 1 -1.946) (width 0.25) (layer "F.Cu") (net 13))
 (segment (start -0.57452 -1.87148) (end -2.12852 -1.87148) (width 0.25) (layer "F.Cu") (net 13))
 (segment (start 2.5 -1.946) (end 2.42548 -1.87148) (width 0.25) (layer "F.Cu") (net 13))
 (segment (start 1.313803 -1.87148) (end 1 -2.185283) (width 0.25) (layer "F.Cu") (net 13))
 (segment (start 2.814803 -1.87148) (end 2.5 -2.186283) (width 0.25) (layer "F.Cu") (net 13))
 (segment (start -2.12852 -1.87148) (end -3.187197 -1.87148) (width 0.25) (layer "F.Cu") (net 13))
 (segment (start 4.001 -1.946) (end 3.92648 -1.87148) (width 0.25) (layer "F.Cu") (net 13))
 (segment (start 2.42548 -1.87148) (end 1.313803 -1.87148) (width 0.25) (layer "F.Cu") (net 13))
 (segment (start -0.5 -3.396) (end -0.5 -1.946) (width 0.25) (layer "F.Cu") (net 13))
 (segment (start 0.92548 -1.87148) (end -0.37148 -1.87148) (width 0.25) (layer "F.Cu") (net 13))
 (segment (start 1 -2.185283) (end 1 -3.396) (width 0.25) (layer "F.Cu") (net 13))
 (segment (start -3.501 -2.185283) (end -3.501 -3.396) (width 0.25) (layer "F.Cu") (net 13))
 (segment (start 2.5 -3.396) (end 2.5 -1.946) (width 0.25) (layer "F.Cu") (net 13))
 (segment (start -3.187197 -1.87148) (end -3.501 -2.185283) (width 0.25) (layer "F.Cu") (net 13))
 (segment (start 3.92648 -1.87148) (end 2.814803 -1.87148) (width 0.25) (layer "F.Cu") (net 13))
 (via (at -2.12852 -0.87148) (size 0.8) (drill 0.4) (layers "F.Cu" "B.Cu") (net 13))
 (segment (start 13 -18) (end 13 -19.1) (width 0.25) (layer "F.Cu") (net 3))
 (segment (start 13 -19.1) (end 13.15 -19.25) (width 0.25) (layer "F.Cu") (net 3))
 (segment (start 3.501 -3.396) (end 3.501 -15.76921) (width 0.25) (layer "F.Cu") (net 3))
 (segment (start 5.73179 -18) (end 13 -18) (width 0.25) (layer "F.Cu") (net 3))
 (segment (start 3.501 -15.76921) (end 5.73179 -18) (width 0.25) (layer "F.Cu") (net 3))
 (segment (start 5.9 -18.803928) (end 5.9 -19.25) (width 0.25) (layer "F.Cu") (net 10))
 (segment (start 3.001 -3.396) (end 3.001 -15.904928) (width 0.25) (layer "F.Cu") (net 10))
 (segment (start 3.001 -15.904928) (end 5.9 -18.803928) (width 0.25) (layer "F.Cu") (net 10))
 (segment (start 4.9 -18.803928) (end 4.9 -19.25) (width 0.25) (layer "F.Cu") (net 11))
 (segment (start 2 -15.903928) (end 4.9 -18.803928) (width 0.25) (layer "F.Cu") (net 11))
 (segment (start 2 -3.396) (end 2 -15.903928) (width 0.25) (layer "F.Cu") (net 11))
 (segment (start 1.5 -3.396) (end 1.5 -8.385717) (width 0.25) (layer "F.Cu") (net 7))
 (segment (start -2.25 -12.135717) (end -2.25 -19.25) (width 0.25) (layer "F.Cu") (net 7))
 (segment (start 1.5 -8.385717) (end -2.25 -12.135717) (width 0.25) (layer "F.Cu") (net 7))
 (segment (start -4.25 -13.185718) (end -4.25 -19.25) (width 0.25) (layer "F.Cu") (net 8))
 (segment (start 0.185718 -8.75) (end -4.25 -13.185718) (width 0.25) (layer "F.Cu") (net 8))
 (segment (start 0.5 -3.396) (end 0.5 -8.75) (width 0.25) (layer "F.Cu") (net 8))
 (segment (start 0.5 -8.75) (end 0.185718 -8.75) (width 0.25) (layer "F.Cu") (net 8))
 (segment (start 0 -8.3) (end -10.95 -19.25) (width 0.25) (layer "F.Cu") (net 5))
 (segment (start 0 -3.396) (end 0 -8.3) (width 0.25) (layer "F.Cu") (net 5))
 (segment (start -1 -7.426804) (end -1 -3.396) (width 0.25) (layer "F.Cu") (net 6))
 (segment (start -12.823196 -19.25) (end -1 -7.426804) (width 0.25) (layer "F.Cu") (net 6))
 (segment (start -12.95 -19.25) (end -12.823196 -19.25) (width 0.25) (layer "F.Cu") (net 6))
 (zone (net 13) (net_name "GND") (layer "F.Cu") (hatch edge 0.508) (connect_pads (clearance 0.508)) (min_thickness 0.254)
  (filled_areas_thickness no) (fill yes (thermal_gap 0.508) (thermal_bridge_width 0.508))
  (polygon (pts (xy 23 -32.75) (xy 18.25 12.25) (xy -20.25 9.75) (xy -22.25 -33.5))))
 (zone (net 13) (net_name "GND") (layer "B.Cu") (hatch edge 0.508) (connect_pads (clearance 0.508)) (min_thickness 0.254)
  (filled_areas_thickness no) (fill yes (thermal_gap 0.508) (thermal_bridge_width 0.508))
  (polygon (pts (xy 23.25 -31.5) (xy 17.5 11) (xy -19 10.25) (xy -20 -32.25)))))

